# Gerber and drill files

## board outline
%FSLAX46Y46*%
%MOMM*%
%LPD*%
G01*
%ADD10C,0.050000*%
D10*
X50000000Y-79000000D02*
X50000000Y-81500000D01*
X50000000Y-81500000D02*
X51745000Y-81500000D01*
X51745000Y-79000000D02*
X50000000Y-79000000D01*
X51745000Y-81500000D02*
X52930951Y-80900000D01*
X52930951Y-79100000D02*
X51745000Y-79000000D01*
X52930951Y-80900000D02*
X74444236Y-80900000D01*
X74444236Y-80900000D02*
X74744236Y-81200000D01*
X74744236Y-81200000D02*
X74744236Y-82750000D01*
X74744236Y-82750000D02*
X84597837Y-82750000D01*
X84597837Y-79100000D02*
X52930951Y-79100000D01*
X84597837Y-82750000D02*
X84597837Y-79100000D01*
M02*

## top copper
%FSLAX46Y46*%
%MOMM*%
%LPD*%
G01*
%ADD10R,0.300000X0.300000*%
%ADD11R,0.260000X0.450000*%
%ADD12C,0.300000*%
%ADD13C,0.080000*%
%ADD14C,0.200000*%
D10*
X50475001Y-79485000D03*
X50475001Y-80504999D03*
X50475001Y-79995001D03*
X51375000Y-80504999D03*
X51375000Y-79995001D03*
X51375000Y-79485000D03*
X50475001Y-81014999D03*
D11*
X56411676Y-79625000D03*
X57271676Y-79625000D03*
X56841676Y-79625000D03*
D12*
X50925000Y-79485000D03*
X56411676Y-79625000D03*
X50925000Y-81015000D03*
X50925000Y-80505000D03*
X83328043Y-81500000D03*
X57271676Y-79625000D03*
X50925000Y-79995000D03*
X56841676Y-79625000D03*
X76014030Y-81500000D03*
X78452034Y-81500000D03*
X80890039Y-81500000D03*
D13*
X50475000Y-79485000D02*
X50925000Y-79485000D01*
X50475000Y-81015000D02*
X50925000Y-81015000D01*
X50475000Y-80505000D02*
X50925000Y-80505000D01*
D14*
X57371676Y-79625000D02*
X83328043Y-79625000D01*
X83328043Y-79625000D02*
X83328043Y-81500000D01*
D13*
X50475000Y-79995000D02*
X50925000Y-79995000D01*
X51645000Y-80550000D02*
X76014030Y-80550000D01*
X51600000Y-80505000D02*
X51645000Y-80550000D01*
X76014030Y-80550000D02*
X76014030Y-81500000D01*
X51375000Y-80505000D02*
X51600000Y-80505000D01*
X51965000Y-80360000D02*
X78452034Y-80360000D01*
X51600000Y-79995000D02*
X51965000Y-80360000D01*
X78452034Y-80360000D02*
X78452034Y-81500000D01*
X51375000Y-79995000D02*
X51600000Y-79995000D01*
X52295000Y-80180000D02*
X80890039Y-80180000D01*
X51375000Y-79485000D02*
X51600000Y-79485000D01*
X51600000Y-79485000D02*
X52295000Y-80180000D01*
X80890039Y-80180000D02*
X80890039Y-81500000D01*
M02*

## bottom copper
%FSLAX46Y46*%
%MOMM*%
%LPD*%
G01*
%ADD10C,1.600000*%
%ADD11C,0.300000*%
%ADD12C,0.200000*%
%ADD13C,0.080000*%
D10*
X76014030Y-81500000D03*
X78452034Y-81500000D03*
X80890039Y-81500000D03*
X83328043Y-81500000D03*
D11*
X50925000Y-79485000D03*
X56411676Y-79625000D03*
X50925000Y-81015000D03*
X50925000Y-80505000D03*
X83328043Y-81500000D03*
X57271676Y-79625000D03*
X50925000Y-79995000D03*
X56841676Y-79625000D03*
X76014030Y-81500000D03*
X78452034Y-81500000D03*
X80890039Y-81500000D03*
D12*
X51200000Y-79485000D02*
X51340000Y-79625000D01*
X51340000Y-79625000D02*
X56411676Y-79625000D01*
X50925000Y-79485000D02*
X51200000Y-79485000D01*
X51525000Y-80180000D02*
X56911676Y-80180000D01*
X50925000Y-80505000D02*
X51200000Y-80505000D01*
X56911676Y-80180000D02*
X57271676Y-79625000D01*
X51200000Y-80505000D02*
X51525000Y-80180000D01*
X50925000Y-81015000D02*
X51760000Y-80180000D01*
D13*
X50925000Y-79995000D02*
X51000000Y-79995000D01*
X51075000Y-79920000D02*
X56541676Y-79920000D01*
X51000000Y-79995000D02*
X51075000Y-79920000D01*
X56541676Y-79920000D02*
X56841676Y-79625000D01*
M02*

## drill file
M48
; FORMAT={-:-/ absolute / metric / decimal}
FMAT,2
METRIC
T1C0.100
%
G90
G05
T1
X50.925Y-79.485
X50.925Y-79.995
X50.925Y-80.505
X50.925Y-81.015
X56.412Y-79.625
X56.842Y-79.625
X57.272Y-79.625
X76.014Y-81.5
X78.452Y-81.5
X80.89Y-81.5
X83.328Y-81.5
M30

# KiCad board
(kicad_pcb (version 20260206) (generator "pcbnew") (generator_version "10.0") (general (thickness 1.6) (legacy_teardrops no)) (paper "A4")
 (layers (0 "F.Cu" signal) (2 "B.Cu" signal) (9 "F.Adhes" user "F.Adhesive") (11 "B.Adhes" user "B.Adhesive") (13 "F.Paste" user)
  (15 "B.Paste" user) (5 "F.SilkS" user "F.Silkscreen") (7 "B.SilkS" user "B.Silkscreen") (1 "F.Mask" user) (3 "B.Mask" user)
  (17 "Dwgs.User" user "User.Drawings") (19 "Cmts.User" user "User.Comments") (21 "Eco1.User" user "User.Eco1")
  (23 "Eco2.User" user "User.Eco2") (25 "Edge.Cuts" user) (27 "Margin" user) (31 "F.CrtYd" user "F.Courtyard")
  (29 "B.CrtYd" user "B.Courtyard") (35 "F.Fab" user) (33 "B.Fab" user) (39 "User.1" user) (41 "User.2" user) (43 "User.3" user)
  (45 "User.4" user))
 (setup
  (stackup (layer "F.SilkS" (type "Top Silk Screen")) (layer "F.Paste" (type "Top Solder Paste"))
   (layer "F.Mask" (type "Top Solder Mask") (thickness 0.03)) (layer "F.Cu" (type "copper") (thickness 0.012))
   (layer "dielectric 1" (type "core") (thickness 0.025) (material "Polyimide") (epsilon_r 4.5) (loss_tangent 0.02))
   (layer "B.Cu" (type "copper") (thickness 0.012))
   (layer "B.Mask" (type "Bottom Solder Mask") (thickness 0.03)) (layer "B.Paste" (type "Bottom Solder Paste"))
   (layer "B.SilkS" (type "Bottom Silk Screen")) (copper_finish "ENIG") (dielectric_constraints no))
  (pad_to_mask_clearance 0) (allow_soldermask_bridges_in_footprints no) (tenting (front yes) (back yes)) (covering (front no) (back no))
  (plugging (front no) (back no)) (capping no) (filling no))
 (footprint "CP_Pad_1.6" (layer "F.Cu") (at 83.328043 81.5)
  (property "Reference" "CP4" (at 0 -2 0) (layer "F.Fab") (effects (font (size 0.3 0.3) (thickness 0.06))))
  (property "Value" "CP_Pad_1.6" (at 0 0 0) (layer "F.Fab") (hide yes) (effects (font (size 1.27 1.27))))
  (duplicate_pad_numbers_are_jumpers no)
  (pad "" smd circle (at -0.346482 -0.346483) (size 0.58 0.58) (layers "B.Paste"))
  (pad "" smd circle (at -0.346482 0.346482) (size 0.58 0.58) (layers "B.Paste"))
  (pad "" smd circle (at 0.346482 -0.346483) (size 0.58 0.58) (layers "B.Paste"))
  (pad "" smd circle (at 0.346482 0.346482) (size 0.58 0.58) (layers "B.Paste"))
  (pad "1" smd circle (at 0 0) (size 1.6 1.6) (layers "B.Cu" "B.Mask") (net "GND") (solder_mask_margin 0.1)))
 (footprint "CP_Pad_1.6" (layer "F.Cu") (at 78.452034 81.5)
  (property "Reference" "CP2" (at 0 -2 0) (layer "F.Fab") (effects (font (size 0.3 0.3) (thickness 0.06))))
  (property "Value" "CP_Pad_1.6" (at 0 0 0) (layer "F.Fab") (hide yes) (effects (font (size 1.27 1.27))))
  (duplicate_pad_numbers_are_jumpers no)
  (pad "" smd circle (at -0.346482 -0.346483) (size 0.58 0.58) (layers "B.Paste"))
  (pad "" smd circle (at -0.346482 0.346482) (size 0.58 0.58) (layers "B.Paste"))
  (pad "" smd circle (at 0.346482 -0.346483) (size 0.58 0.58) (layers "B.Paste"))
  (pad "" smd circle (at 0.346482 0.346482) (size 0.58 0.58) (layers "B.Paste"))
  (pad "1" smd circle (at 0 0) (size 1.6 1.6) (layers "B.Cu" "B.Mask") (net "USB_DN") (solder_mask_margin 0.1)))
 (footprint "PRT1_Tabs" (layer "F.Cu") (at 56.841676 79.625)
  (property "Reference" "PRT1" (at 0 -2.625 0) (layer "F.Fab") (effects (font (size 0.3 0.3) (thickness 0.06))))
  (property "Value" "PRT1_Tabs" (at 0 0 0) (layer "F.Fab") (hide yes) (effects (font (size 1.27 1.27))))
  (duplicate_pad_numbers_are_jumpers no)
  (pad "1" smd rect (at -0.43 0) (size 0.26 0.45) (layers "F.Cu" "F.Mask") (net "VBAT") (solder_mask_margin 0.05) (thermal_bridge_angle 45))
  (pad "2" smd rect (at 0.43 0) (size 0.26 0.45) (layers "F.Cu" "F.Mask") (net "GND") (solder_mask_margin 0.05) (thermal_bridge_angle 45))
  (pad "3" smd rect (at 0 0) (size 0.26 0.45) (layers "F.Cu" "F.Mask") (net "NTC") (solder_mask_margin 0.05) (thermal_bridge_angle 45)))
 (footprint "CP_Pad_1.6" (layer "F.Cu") (at 80.890039 81.5)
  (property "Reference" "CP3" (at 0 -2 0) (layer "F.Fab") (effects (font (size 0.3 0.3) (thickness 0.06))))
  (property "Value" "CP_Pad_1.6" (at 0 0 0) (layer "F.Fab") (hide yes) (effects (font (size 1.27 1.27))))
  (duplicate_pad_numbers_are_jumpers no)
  (pad "" smd circle (at -0.346483 -0.346483) (size 0.58 0.58) (layers "B.Paste"))
  (pad "" smd circle (at -0.346483 0.346482) (size 0.58 0.58) (layers "B.Paste"))
  (pad "" smd circle (at 0.346482 -0.346483) (size 0.58 0.58) (layers "B.Paste"))
  (pad "" smd circle (at 0.346482 0.346482) (size 0.58 0.58) (layers "B.Paste"))
  (pad "1" smd circle (at 0 0) (size 1.6 1.6) (layers "B.Cu" "B.Mask") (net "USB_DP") (solder_mask_margin 0.1)))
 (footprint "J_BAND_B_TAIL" (layer "F.Cu") (at 50.9 80.25)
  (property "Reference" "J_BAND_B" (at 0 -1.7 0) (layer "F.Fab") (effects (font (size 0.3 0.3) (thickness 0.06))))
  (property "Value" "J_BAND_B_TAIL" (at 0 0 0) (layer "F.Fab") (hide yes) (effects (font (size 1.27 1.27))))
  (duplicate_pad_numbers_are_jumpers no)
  (pad "1" smd rect (at -0.424999 -0.765) (size 0.3 0.3) (layers "F.Cu" "F.Mask") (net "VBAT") (solder_mask_margin 0.05)
   (thermal_bridge_angle 45))
  (pad "2" smd rect (at -0.424999 0.254999) (size 0.3 0.3) (layers "F.Cu" "F.Mask") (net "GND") (solder_mask_margin 0.05)
   (thermal_bridge_angle 45))
  (pad "3" smd rect (at -0.424999 -0.254999) (size 0.3 0.3) (layers "F.Cu" "F.Mask") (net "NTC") (solder_mask_margin 0.05)
   (thermal_bridge_angle 45))
  (pad "4" smd rect (at 0.475 0.254999) (size 0.3 0.3) (layers "F.Cu" "F.Mask") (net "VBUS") (solder_mask_margin 0.05)
   (thermal_bridge_angle 45))
  (pad "5" smd rect (at 0.475 -0.254999) (size 0.3 0.3) (layers "F.Cu" "F.Mask") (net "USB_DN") (solder_mask_margin 0.05)
   (thermal_bridge_angle 45))
  (pad "6" smd rect (at 0.475 -0.765) (size 0.3 0.3) (layers "F.Cu" "F.Mask") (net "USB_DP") (solder_mask_margin 0.05)
   (thermal_bridge_angle 45))
  (pad "7" smd rect (at -0.424999 0.764999) (size 0.3 0.3) (layers "F.Cu" "F.Mask") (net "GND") (solder_mask_margin 0.05)
   (thermal_bridge_angle 45)))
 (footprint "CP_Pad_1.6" (layer "F.Cu") (at 76.01403 81.5)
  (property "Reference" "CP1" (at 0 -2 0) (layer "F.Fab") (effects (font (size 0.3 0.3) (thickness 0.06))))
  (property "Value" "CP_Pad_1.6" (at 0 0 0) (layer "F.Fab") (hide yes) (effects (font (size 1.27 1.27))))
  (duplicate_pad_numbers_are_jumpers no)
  (pad "" smd circle (at -0.346483 0.346482) (size 0.58 0.58) (layers "B.Paste"))
  (pad "" smd circle (at 0.346482 -0.346483) (size 0.58 0.58) (layers "B.Paste"))
  (pad "" smd circle (at 0.346482 0.346482) (size 0.58 0.58) (layers "B.Paste"))
  (pad "1" smd circle (at 0 0) (size 1.6 1.6) (layers "B.Cu" "B.Mask") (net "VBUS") (solder_mask_margin 0.1)))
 (gr_line (start 50 79) (end 50 81.5) (stroke (width 0.05) (type default)) (layer "Edge.Cuts"))
 (gr_line (start 50 81.5) (end 51.745 81.5) (stroke (width 0.05) (type default)) (layer "Edge.Cuts"))
 (gr_line (start 51.745 79) (end 50 79) (stroke (width 0.05) (type default)) (layer "Edge.Cuts"))
 (gr_line (start 51.745 81.5) (end 52.930951 80.9) (stroke (width 0.05) (type default)) (layer "Edge.Cuts"))
 (gr_line (start 52.930951 79.1) (end 51.745 79) (stroke (width 0.05) (type default)) (layer "Edge.Cuts"))
 (gr_line (start 52.930951 80.9) (end 74.444236 80.9) (stroke (width 0.05) (type default)) (layer "Edge.Cuts"))
 (gr_line (start 74.444236 80.9) (end 74.744236 81.2) (stroke (width 0.05) (type default)) (layer "Edge.Cuts"))
 (gr_line (start 74.744236 81.2) (end 74.744236 82.75) (stroke (width 0.05) (type default)) (layer "Edge.Cuts"))
 (gr_line (start 74.744236 82.75) (end 84.597837 82.75) (stroke (width 0.05) (type default)) (layer "Edge.Cuts"))
 (gr_line (start 84.597837 79.1) (end 52.930951 79.1) (stroke (width 0.05) (type default)) (layer "Edge.Cuts"))
 (gr_line (start 84.597837 82.75) (end 84.597837 79.1) (stroke (width 0.05) (type default)) (layer "Edge.Cuts"))
 (segment (start 50.475 81.015) (end 50.925 81.015) (width 0.08) (layer "F.Cu") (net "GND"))
 (segment (start 50.475 80.505) (end 50.925 80.505) (width 0.08) (layer "F.Cu") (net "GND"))
 (segment (start 83.328043 79.625) (end 83.328043 81.5) (width 0.2) (layer "F.Cu") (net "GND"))
 (segment (start 57.371676 79.625) (end 83.328043 79.625) (width 0.2) (layer "F.Cu") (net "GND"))
 (via (at 50.925 80.505) (size 0.3) (drill 0.1) (layers "F.Cu" "B.Cu") (tenting (front yes) (back yes)) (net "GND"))
 (via (at 83.328043 81.5) (size 0.3) (drill 0.1) (layers "F.Cu" "B.Cu") (tenting (front yes) (back yes)) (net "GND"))
 (via (at 57.271676 79.625) (size 0.3) (drill 0.1) (layers "F.Cu" "B.Cu") (tenting (front yes) (back yes)) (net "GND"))
 (via (at 50.925 81.015) (size 0.3) (drill 0.1) (layers "F.Cu" "B.Cu") (tenting (front yes) (back yes)) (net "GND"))
 (segment (start 50.925 80.505) (end 51.2 80.505) (width 0.2) (layer "B.Cu") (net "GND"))
 (segment (start 50.925 81.015) (end 51.76 80.18) (width 0.2) (layer "B.Cu") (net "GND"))
 (segment (start 51.2 80.505) (end 51.525 80.18) (width 0.2) (layer "B.Cu") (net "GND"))
 (segment (start 51.525 80.18) (end 56.911676 80.18) (width 0.2) (layer "B.Cu") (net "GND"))
 (segment (start 56.911676 80.18) (end 57.271676 79.625) (width 0.2) (layer "B.Cu") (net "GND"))
 (segment (start 78.452034 80.36) (end 78.452034 81.5) (width 0.08) (layer "F.Cu") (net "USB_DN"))
 (segment (start 51.965 80.36) (end 78.452034 80.36) (width 0.08) (layer "F.Cu") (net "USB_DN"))
 (segment (start 51.6 79.995) (end 51.965 80.36) (width 0.08) (layer "F.Cu") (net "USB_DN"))
 (segment (start 51.375 79.995) (end 51.6 79.995) (width 0.08) (layer "F.Cu") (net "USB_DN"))
 (via (at 78.452034 81.5) (size 0.3) (drill 0.1) (layers "F.Cu" "B.Cu") (tenting (front yes) (back yes)) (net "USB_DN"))
 (segment (start 50.475 79.485) (end 50.925 79.485) (width 0.08) (layer "F.Cu") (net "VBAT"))
 (via (at 56.411676 79.625) (size 0.3) (drill 0.1) (layers "F.Cu" "B.Cu") (tenting (front yes) (back yes)) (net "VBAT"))
 (via (at 50.925 79.485) (size 0.3) (drill 0.1) (layers "F.Cu" "B.Cu") (tenting (front yes) (back yes)) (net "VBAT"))
 (segment (start 51.34 79.625) (end 56.411676 79.625) (width 0.2) (layer "B.Cu") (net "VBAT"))
 (segment (start 51.2 79.485) (end 51.34 79.625) (width 0.2) (layer "B.Cu") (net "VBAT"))
 (segment (start 50.925 79.485) (end 51.2 79.485) (width 0.2) (layer "B.Cu") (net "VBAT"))
 (segment (start 50.475 79.995) (end 50.925 79.995) (width 0.08) (layer "F.Cu") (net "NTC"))
 (via (at 50.925 79.995) (size 0.3) (drill 0.1) (layers "F.Cu" "B.Cu") (tenting (front yes) (back yes)) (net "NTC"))
 (via (at 56.841676 79.625) (size 0.3) (drill 0.1) (layers "F.Cu" "B.Cu") (tenting (front yes) (back yes)) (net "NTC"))
 (segment (start 56.541676 79.92) (end 56.841676 79.625) (width 0.08) (layer "B.Cu") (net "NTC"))
 (segment (start 51.075 79.92) (end 56.541676 79.92) (width 0.08) (layer "B.Cu") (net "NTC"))
 (segment (start 51 79.995) (end 51.075 79.92) (width 0.08) (layer "B.Cu") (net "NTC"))
 (segment (start 50.925 79.995) (end 51 79.995) (width 0.08) (layer "B.Cu") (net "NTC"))
 (segment (start 51.6 79.485) (end 52.295 80.18) (width 0.08) (layer "F.Cu") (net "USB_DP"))
 (segment (start 51.375 79.485) (end 51.6 79.485) (width 0.08) (layer "F.Cu") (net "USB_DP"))
 (segment (start 52.295 80.18) (end 80.890039 80.18) (width 0.08) (layer "F.Cu") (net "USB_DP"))
 (segment (start 80.890039 80.18) (end 80.890039 81.5) (width 0.08) (layer "F.Cu") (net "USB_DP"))
 (via (at 80.890039 81.5) (size 0.3) (drill 0.1) (layers "F.Cu" "B.Cu") (tenting (front yes) (back yes)) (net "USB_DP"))
 (segment (start 76.01403 80.55) (end 76.01403 81.5) (width 0.08) (layer "F.Cu") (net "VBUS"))
 (segment (start 51.6 80.505) (end 51.645 80.55) (width 0.08) (layer "F.Cu") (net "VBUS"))
 (segment (start 51.375 80.505) (end 51.6 80.505) (width 0.08) (layer "F.Cu") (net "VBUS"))
 (segment (start 51.645 80.55) (end 76.01403 80.55) (width 0.08) (layer "F.Cu") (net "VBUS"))
 (via (at 76.01403 81.5) (size 0.3) (drill 0.1) (layers "F.Cu" "B.Cu") (tenting (front yes) (back yes)) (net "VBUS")))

